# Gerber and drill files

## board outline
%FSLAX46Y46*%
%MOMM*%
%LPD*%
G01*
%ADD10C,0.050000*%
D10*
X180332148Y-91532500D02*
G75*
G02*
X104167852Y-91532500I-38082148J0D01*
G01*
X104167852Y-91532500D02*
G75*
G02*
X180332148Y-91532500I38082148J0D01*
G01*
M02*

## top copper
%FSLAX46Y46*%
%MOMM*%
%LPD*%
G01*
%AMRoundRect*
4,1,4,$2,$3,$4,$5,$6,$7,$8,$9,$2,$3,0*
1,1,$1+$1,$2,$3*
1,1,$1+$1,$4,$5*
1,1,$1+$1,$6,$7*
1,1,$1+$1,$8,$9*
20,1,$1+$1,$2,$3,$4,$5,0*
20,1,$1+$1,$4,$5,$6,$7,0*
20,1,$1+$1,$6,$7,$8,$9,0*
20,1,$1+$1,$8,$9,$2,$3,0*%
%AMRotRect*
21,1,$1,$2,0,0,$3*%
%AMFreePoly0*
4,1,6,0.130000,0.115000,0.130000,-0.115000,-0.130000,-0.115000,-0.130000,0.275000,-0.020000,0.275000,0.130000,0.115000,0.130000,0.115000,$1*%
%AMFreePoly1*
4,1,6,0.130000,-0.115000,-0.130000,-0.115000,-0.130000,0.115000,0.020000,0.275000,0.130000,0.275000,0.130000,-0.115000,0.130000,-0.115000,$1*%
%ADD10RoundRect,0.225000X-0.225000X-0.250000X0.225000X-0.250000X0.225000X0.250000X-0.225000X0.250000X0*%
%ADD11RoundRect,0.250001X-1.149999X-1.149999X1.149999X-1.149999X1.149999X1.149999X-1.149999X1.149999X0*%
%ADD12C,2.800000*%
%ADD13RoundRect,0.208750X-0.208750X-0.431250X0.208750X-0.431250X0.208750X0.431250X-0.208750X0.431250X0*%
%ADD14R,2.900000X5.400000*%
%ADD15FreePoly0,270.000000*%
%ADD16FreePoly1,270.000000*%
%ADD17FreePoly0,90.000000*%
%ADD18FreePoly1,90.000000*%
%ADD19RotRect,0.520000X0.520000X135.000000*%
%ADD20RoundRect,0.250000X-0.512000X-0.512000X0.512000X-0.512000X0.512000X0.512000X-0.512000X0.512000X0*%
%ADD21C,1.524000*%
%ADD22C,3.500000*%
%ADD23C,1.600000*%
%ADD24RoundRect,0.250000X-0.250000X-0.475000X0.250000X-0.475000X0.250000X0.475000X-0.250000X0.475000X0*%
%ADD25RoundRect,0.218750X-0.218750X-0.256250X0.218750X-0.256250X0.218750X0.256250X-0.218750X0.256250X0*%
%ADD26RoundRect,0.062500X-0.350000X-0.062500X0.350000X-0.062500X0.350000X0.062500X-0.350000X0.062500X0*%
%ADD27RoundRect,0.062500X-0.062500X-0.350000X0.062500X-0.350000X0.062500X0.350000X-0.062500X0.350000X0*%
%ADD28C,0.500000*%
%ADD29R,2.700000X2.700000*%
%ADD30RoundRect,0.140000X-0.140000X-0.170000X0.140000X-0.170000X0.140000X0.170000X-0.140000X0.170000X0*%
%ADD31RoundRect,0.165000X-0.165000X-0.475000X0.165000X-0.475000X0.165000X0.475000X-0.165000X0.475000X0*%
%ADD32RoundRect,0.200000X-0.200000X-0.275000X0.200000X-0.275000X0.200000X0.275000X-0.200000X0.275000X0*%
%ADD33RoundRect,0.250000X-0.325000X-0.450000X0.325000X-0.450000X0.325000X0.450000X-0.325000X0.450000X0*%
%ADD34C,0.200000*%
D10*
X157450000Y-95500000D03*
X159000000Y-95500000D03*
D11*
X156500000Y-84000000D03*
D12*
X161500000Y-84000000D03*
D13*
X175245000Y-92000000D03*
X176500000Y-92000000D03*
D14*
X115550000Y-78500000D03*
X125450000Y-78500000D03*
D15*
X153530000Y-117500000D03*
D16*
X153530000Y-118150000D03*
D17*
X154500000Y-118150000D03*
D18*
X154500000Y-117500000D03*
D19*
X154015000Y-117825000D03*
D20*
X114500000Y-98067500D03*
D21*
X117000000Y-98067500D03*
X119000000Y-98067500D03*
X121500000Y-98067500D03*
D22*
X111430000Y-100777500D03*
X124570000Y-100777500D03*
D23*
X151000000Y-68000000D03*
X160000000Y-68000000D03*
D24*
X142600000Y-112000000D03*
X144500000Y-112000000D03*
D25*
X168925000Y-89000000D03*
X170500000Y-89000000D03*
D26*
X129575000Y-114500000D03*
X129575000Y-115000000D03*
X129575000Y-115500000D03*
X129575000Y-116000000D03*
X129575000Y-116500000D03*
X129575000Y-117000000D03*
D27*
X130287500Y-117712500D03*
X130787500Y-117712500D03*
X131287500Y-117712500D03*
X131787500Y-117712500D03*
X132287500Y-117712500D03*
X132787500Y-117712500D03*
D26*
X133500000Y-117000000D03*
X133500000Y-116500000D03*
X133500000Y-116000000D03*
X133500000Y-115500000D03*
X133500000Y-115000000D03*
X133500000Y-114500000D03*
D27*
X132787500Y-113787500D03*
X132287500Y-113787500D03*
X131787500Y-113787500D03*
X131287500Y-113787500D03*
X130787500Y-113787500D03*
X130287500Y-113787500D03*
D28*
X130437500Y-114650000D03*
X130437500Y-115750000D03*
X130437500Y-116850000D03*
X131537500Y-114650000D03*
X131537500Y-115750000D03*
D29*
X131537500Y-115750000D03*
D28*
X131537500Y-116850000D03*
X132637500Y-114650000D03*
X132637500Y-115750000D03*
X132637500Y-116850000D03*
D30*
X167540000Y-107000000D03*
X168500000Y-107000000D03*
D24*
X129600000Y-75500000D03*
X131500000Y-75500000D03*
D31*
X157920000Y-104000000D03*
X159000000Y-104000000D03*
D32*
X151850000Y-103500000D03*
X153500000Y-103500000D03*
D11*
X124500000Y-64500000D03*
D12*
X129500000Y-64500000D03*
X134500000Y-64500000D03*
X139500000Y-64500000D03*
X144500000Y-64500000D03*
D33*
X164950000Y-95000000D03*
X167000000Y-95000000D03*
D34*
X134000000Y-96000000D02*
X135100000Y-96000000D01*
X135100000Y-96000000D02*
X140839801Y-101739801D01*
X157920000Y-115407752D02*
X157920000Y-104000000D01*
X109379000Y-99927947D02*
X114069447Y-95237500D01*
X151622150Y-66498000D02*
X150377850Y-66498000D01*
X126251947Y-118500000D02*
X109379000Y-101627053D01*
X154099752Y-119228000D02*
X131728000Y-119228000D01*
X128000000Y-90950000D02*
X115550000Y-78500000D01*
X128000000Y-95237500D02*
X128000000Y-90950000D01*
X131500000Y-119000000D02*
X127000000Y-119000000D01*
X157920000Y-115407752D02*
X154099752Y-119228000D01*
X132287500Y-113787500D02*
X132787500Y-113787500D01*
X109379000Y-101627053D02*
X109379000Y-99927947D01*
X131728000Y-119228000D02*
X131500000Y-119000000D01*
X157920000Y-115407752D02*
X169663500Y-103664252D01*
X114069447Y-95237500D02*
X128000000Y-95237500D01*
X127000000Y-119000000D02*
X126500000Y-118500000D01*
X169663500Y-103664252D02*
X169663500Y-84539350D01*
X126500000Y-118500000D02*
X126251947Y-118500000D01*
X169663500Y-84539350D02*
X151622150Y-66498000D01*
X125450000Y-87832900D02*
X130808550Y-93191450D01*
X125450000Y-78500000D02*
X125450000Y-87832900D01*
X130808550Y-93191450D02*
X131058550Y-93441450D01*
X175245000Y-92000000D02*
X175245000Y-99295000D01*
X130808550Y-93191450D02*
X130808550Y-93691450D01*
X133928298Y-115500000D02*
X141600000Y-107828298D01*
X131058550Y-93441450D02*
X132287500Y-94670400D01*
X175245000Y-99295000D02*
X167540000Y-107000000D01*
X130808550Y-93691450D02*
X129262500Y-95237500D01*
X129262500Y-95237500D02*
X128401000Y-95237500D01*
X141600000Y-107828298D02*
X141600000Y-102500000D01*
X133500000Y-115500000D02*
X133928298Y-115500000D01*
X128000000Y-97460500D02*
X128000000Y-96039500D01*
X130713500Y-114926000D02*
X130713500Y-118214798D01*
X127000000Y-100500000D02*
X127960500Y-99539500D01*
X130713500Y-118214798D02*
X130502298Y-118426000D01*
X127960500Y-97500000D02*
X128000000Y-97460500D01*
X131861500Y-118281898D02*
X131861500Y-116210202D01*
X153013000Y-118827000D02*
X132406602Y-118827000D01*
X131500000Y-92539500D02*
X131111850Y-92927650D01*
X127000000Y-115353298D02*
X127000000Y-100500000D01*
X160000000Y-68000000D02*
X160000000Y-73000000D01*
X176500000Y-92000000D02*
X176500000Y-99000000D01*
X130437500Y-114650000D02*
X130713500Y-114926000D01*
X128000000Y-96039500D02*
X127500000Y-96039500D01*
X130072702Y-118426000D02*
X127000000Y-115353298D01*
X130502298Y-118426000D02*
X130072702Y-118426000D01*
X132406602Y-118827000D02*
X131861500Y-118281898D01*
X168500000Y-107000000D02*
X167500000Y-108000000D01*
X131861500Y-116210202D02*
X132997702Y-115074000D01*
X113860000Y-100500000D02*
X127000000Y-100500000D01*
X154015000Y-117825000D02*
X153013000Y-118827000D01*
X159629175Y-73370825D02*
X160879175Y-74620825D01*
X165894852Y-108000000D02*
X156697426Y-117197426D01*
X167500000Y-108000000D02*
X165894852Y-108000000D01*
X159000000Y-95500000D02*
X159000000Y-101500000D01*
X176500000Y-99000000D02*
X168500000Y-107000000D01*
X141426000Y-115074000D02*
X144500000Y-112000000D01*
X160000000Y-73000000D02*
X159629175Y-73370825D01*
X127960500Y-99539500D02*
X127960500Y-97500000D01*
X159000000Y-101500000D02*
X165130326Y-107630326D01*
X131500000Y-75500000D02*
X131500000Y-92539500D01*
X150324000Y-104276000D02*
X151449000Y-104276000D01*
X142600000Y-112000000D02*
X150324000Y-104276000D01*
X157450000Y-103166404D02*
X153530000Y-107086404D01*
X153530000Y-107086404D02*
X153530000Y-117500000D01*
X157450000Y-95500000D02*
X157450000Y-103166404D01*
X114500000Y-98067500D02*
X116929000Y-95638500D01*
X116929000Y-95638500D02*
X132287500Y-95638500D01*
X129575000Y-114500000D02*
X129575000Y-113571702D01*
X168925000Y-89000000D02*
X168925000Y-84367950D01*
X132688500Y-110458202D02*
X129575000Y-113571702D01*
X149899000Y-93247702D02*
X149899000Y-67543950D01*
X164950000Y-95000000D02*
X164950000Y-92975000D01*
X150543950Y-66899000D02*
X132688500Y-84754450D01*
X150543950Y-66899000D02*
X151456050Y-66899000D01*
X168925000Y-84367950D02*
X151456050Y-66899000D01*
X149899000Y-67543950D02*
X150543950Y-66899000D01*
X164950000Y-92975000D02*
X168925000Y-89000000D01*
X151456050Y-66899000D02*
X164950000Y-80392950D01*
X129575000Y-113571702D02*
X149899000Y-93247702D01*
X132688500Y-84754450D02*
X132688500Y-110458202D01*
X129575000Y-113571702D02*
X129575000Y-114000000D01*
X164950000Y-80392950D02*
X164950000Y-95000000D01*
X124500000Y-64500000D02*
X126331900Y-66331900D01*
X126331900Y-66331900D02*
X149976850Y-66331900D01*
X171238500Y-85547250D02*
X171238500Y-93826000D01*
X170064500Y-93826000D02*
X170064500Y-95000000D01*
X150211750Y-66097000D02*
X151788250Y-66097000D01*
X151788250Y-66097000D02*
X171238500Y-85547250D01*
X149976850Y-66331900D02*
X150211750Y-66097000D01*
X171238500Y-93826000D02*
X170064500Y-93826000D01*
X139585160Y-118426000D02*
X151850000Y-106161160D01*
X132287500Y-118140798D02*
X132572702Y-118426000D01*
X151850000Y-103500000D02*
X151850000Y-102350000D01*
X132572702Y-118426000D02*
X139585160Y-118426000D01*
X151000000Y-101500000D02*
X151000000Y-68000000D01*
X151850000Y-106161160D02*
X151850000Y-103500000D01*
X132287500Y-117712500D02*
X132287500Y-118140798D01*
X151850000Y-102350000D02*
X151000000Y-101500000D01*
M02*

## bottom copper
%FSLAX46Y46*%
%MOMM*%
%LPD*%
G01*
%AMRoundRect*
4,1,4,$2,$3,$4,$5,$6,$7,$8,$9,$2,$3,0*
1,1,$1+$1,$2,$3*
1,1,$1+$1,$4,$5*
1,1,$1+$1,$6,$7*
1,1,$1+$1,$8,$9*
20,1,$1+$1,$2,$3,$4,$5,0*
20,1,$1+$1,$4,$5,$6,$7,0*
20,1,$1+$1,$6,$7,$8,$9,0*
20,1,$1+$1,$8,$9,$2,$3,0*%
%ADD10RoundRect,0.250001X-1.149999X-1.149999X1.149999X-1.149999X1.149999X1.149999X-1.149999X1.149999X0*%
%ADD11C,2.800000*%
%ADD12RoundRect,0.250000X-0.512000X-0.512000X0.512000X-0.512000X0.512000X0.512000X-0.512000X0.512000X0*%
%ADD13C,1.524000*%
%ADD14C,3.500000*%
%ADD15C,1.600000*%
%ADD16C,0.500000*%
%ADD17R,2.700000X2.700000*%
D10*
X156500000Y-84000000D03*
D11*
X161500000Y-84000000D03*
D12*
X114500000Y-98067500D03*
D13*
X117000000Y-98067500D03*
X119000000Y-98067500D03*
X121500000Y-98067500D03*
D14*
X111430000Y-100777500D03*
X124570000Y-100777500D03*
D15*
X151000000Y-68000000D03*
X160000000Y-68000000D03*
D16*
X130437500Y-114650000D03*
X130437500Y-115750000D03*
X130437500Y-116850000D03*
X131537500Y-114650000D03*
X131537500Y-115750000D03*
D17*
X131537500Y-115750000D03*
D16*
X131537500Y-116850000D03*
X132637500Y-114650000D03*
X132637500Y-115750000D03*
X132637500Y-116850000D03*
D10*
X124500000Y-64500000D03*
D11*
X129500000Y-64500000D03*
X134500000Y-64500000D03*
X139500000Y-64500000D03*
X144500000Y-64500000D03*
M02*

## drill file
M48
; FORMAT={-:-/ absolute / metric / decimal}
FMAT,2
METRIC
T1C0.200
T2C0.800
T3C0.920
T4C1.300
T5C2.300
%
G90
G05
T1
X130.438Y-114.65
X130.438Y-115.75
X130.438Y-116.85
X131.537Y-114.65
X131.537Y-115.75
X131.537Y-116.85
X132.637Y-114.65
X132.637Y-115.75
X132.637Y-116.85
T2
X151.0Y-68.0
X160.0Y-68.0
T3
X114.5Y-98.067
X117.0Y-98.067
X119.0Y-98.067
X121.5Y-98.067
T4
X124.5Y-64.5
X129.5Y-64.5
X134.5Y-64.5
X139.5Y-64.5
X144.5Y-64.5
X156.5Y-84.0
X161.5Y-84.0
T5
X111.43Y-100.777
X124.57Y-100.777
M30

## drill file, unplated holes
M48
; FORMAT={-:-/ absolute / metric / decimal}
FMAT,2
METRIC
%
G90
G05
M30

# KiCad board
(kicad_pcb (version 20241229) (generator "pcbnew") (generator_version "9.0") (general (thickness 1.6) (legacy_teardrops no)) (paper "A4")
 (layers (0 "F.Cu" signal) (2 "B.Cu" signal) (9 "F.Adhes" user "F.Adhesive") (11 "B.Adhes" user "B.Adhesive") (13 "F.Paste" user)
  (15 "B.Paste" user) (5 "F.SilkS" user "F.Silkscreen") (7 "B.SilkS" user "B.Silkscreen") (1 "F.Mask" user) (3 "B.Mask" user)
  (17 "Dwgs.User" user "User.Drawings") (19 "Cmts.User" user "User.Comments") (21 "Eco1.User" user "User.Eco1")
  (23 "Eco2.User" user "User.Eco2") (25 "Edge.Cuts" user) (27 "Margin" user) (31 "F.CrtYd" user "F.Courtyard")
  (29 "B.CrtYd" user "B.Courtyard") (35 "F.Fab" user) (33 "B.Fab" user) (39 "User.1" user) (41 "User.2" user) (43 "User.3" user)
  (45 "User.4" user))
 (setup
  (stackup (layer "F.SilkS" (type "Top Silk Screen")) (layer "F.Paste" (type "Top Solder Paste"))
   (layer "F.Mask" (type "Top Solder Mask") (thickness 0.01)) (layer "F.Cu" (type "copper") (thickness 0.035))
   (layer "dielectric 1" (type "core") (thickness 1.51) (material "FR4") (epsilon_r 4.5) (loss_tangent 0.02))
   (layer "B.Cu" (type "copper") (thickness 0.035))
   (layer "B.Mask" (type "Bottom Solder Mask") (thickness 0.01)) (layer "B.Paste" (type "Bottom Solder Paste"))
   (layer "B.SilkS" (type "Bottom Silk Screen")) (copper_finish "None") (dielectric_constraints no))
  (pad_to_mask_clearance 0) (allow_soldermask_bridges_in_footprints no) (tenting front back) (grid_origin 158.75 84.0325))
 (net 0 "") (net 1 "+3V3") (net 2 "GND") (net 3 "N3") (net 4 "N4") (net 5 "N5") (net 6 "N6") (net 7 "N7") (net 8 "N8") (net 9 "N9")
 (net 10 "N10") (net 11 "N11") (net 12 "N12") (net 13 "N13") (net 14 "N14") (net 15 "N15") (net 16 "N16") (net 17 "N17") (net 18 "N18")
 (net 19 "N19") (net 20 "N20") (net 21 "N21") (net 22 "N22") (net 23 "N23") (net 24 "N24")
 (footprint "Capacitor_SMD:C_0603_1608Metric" (layer "F.Cu") (at 158.225 95.5)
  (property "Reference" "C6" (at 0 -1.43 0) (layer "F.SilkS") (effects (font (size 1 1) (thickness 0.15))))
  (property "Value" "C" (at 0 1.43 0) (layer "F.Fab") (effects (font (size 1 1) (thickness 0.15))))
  (pad "1" smd roundrect (at -0.775 0) (size 0.9 0.95) (layers "F.Cu" "F.Mask" "F.Paste") (roundrect_rratio 0.25) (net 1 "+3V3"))
  (pad "2" smd roundrect (at 0.775 0) (size 0.9 0.95) (layers "F.Cu" "F.Mask" "F.Paste") (roundrect_rratio 0.25) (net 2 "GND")))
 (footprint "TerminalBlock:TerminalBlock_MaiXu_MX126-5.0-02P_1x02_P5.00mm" (layer "F.Cu") (at 156.5 84)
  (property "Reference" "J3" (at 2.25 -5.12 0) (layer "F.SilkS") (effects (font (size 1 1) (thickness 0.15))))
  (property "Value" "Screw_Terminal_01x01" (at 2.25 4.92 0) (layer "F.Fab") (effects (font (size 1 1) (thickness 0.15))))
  (pad "1" thru_hole roundrect (at 0 0) (size 2.8 2.8) (drill 1.3) (layers "*.Cu" "*.Mask") (remove_unused_layers no)
   (roundrect_rratio 0.089286) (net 2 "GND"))
  (pad "2" thru_hole circle (at 5 0) (size 2.8 2.8) (drill 1.3) (layers "*.Cu" "*.Mask") (remove_unused_layers no)))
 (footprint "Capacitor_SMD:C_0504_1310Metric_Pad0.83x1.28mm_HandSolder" (layer "F.Cu") (at 175.8725 92)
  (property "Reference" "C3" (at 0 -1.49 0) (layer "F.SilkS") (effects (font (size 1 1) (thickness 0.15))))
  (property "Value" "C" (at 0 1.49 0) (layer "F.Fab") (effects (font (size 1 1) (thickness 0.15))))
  (pad "1" smd roundrect (at -0.6275 0) (size 0.835 1.28) (layers "F.Cu" "F.Mask" "F.Paste") (roundrect_rratio 0.25) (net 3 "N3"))
  (pad "2" smd roundrect (at 0.6275 0) (size 0.835 1.28) (layers "F.Cu" "F.Mask" "F.Paste") (roundrect_rratio 0.25) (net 2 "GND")))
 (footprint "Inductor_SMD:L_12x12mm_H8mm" (layer "F.Cu") (at 120.5 78.5)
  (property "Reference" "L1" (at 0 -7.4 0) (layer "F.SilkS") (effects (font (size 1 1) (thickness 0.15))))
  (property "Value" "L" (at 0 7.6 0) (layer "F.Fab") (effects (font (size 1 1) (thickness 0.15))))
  (pad "1" smd rect (at -4.95 0) (size 2.9 5.4) (layers "F.Cu" "F.Mask" "F.Paste") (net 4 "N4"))
  (pad "2" smd rect (at 4.95 0) (size 2.9 5.4) (layers "F.Cu" "F.Mask" "F.Paste") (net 3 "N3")))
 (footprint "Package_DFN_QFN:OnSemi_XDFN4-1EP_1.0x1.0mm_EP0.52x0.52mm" (layer "F.Cu") (at 154.015 117.825)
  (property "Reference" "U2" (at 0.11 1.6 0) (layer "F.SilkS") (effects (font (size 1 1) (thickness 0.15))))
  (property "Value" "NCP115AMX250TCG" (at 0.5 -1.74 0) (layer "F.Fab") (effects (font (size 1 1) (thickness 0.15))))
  (pad "1" smd custom (at -0.485 -0.325 270) (size 0.26 0.23) (layers "F.Cu" "F.Mask" "F.Paste") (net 1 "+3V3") (zone_connect 0)
   (thermal_bridge_angle 45) (options (clearance outline) (anchor rect)) (primitives))
  (pad "2" smd custom (at -0.485 0.325 270) (size 0.26 0.23) (layers "F.Cu" "F.Mask" "F.Paste") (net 2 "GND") (zone_connect 0)
   (thermal_bridge_angle 45) (options (clearance outline) (anchor rect)) (primitives))
  (pad "3" smd custom (at 0.485 0.325 90) (size 0.26 0.23) (layers "F.Cu" "F.Mask" "F.Paste") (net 3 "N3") (zone_connect 0)
   (thermal_bridge_angle 45) (options (clearance outline) (anchor rect)) (primitives))
  (pad "4" smd custom (at 0.485 -0.325 90) (size 0.26 0.23) (layers "F.Cu" "F.Mask" "F.Paste") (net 3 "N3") (zone_connect 0)
   (thermal_bridge_angle 45) (options (clearance outline) (anchor rect)) (primitives))
  (pad "5" smd rect (at 0 0 135) (size 0.52 0.52) (layers "F.Cu" "F.Mask" "F.Paste") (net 2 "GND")))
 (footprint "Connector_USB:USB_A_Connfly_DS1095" (layer "F.Cu") (at 114.5 98.0675)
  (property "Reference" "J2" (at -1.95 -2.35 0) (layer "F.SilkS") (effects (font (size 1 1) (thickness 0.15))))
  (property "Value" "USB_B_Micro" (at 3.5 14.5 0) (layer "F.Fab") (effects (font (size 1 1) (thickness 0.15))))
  (pad "1" thru_hole roundrect (at 0 0) (size 1.524 1.524) (drill 0.92) (layers "*.Cu" "*.Mask") (remove_unused_layers no)
   (roundrect_rratio 0.1640419948) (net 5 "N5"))
  (pad "2" thru_hole circle (at 2.5 0) (size 1.524 1.524) (drill 0.92) (layers "*.Cu" "*.Mask") (remove_unused_layers no) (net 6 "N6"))
  (pad "3" thru_hole circle (at 4.5 0) (size 1.524 1.524) (drill 0.92) (layers "*.Cu" "*.Mask") (remove_unused_layers no) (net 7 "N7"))
  (pad "4" thru_hole circle (at 7 0) (size 1.524 1.524) (drill 0.92) (layers "*.Cu" "*.Mask") (remove_unused_layers no) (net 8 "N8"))
  (pad "5" thru_hole circle (at -3.07 2.71) (size 3.5 3.5) (drill 2.3) (layers "*.Cu" "*.Mask") (remove_unused_layers no) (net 2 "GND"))
  (pad "5" thru_hole circle (at 10.07 2.71) (size 3.5 3.5) (drill 2.3) (layers "*.Cu" "*.Mask") (remove_unused_layers no) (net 2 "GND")))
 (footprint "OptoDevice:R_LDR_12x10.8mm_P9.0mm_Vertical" (layer "F.Cu") (at 151 68)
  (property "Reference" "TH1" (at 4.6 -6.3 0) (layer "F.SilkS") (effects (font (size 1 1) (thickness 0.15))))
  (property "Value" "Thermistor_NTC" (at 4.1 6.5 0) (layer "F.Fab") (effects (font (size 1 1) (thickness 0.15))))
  (pad "1" thru_hole circle (at 0 0) (size 1.6 1.6) (drill 0.8) (layers "*.Cu" "*.Mask") (remove_unused_layers no) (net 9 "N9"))
  (pad "2" thru_hole circle (at 9 0) (size 1.6 1.6) (drill 0.8) (layers "*.Cu" "*.Mask") (remove_unused_layers no) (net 2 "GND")))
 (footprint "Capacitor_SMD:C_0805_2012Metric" (layer "F.Cu") (at 143.55 112)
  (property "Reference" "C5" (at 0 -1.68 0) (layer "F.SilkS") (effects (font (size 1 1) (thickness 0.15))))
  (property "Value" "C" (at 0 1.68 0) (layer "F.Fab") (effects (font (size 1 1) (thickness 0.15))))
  (pad "1" smd roundrect (at -0.95 0) (size 1 1.45) (layers "F.Cu" "F.Mask" "F.Paste") (roundrect_rratio 0.25) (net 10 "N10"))
  (pad "2" smd roundrect (at 0.95 0) (size 1 1.45) (layers "F.Cu" "F.Mask" "F.Paste") (roundrect_rratio 0.25) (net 2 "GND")))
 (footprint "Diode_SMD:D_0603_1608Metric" (layer "F.Cu") (at 169.7125 89)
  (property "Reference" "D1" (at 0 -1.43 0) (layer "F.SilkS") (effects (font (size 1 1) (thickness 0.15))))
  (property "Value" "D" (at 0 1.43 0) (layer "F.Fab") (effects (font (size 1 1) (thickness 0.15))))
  (pad "1" smd roundrect (at -0.7875 0) (size 0.875 0.95) (layers "F.Cu" "F.Mask" "F.Paste") (roundrect_rratio 0.25) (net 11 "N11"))
  (pad "2" smd roundrect (at 0.7875 0) (size 0.875 0.95) (layers "F.Cu" "F.Mask" "F.Paste") (roundrect_rratio 0.25) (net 5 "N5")))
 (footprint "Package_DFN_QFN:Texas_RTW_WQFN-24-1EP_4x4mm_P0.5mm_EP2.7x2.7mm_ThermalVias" (layer "F.Cu") (at 131.5375 115.75)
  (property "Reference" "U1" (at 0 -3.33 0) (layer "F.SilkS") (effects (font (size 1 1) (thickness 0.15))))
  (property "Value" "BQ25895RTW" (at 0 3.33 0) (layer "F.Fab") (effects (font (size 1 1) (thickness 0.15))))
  (pad "" smd roundrect (at -0.675 -0.675) (size 1.13 1.13) (layers "F.Paste") (roundrect_rratio 0.221239))
  (pad "" smd roundrect (at -0.675 0.675) (size 1.13 1.13) (layers "F.Paste") (roundrect_rratio 0.221239))
  (pad "" smd roundrect (at 0.675 -0.675) (size 1.13 1.13) (layers "F.Paste") (roundrect_rratio 0.221239))
  (pad "" smd roundrect (at 0.675 0.675) (size 1.13 1.13) (layers "F.Paste") (roundrect_rratio 0.221239))
  (pad "1" smd roundrect (at -1.9625 -1.25) (size 0.825 0.25) (layers "F.Cu" "F.Mask" "F.Paste") (roundrect_rratio 0.25) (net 11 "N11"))
  (pad "2" smd roundrect (at -1.9625 -0.75) (size 0.825 0.25) (layers "F.Cu" "F.Mask" "F.Paste") (roundrect_rratio 0.25) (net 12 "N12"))
  (pad "3" smd roundrect (at -1.9625 -0.25) (size 0.825 0.25) (layers "F.Cu" "F.Mask" "F.Paste") (roundrect_rratio 0.25) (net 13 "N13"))
  (pad "4" smd roundrect (at -1.9625 0.25) (size 0.825 0.25) (layers "F.Cu" "F.Mask" "F.Paste") (roundrect_rratio 0.25) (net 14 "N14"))
  (pad "5" smd roundrect (at -1.9625 0.75) (size 0.825 0.25) (layers "F.Cu" "F.Mask" "F.Paste") (roundrect_rratio 0.25) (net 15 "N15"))
  (pad "6" smd roundrect (at -1.9625 1.25) (size 0.825 0.25) (layers "F.Cu" "F.Mask" "F.Paste") (roundrect_rratio 0.25) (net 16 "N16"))
  (pad "7" smd roundrect (at -1.25 1.9625) (size 0.25 0.825) (layers "F.Cu" "F.Mask" "F.Paste") (roundrect_rratio 0.25) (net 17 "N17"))
  (pad "8" smd roundrect (at -0.75 1.9625) (size 0.25 0.825) (layers "F.Cu" "F.Mask" "F.Paste") (roundrect_rratio 0.25) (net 2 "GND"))
  (pad "9" smd roundrect (at -0.25 1.9625) (size 0.25 0.825) (layers "F.Cu" "F.Mask" "F.Paste") (roundrect_rratio 0.25) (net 2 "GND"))
  (pad "10" smd roundrect (at 0.25 1.9625) (size 0.25 0.825) (layers "F.Cu" "F.Mask" "F.Paste") (roundrect_rratio 0.25) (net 2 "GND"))
  (pad "11" smd roundrect (at 0.75 1.9625) (size 0.25 0.825) (layers "F.Cu" "F.Mask" "F.Paste") (roundrect_rratio 0.25) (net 9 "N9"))
  (pad "12" smd roundrect (at 1.25 1.9625) (size 0.25 0.825) (layers "F.Cu" "F.Mask" "F.Paste") (roundrect_rratio 0.25) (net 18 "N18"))
  (pad "13" smd roundrect (at 1.9625 1.25) (size 0.825 0.25) (layers "F.Cu" "F.Mask" "F.Paste") (roundrect_rratio 0.25) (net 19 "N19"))
  (pad "14" smd roundrect (at 1.9625 0.75) (size 0.825 0.25) (layers "F.Cu" "F.Mask" "F.Paste") (roundrect_rratio 0.25) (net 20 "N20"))
  (pad "15" smd roundrect (at 1.9625 0.25) (size 0.825 0.25) (layers "F.Cu" "F.Mask" "F.Paste") (roundrect_rratio 0.25) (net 3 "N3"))
  (pad "16" smd roundrect (at 1.9625 -0.25) (size 0.825 0.25) (layers "F.Cu" "F.Mask" "F.Paste") (roundrect_rratio 0.25) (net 3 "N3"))
  (pad "17" smd roundrect (at 1.9625 -0.75) (size 0.825 0.25) (layers "F.Cu" "F.Mask" "F.Paste") (roundrect_rratio 0.25) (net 2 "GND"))
  (pad "18" smd roundrect (at 1.9625 -1.25) (size 0.825 0.25) (layers "F.Cu" "F.Mask" "F.Paste") (roundrect_rratio 0.25) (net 2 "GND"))
  (pad "19" smd roundrect (at 1.25 -1.9625) (size 0.25 0.825) (layers "F.Cu" "F.Mask" "F.Paste") (roundrect_rratio 0.25) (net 4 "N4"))
  (pad "20" smd roundrect (at 0.75 -1.9625) (size 0.25 0.825) (layers "F.Cu" "F.Mask" "F.Paste") (roundrect_rratio 0.25) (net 4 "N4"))
  (pad "21" smd roundrect (at 0.25 -1.9625) (size 0.25 0.825) (layers "F.Cu" "F.Mask" "F.Paste") (roundrect_rratio 0.25) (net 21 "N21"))
  (pad "22" smd roundrect (at -0.25 -1.9625) (size 0.25 0.825) (layers "F.Cu" "F.Mask" "F.Paste") (roundrect_rratio 0.25) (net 10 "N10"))
  (pad "23" smd roundrect (at -0.75 -1.9625) (size 0.25 0.825) (layers "F.Cu" "F.Mask" "F.Paste") (roundrect_rratio 0.25) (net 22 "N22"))
  (pad "24" smd roundrect (at -1.25 -1.9625) (size 0.25 0.825) (layers "F.Cu" "F.Mask" "F.Paste") (roundrect_rratio 0.25) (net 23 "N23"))
  (pad "25" thru_hole circle (at -1.1 -1.1) (size 0.5 0.5) (drill 0.2) (layers "*.Cu") (remove_unused_layers no) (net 2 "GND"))
  (pad "25" thru_hole circle (at -1.1 0) (size 0.5 0.5) (drill 0.2) (layers "*.Cu") (remove_unused_layers no) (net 2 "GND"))
  (pad "25" thru_hole circle (at -1.1 1.1) (size 0.5 0.5) (drill 0.2) (layers "*.Cu") (remove_unused_layers no) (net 2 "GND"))
  (pad "25" thru_hole circle (at 0 -1.1) (size 0.5 0.5) (drill 0.2) (layers "*.Cu") (remove_unused_layers no) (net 2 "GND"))
  (pad "25" thru_hole circle (at 0 0) (size 0.5 0.5) (drill 0.2) (layers "*.Cu") (remove_unused_layers no) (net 2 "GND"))
  (pad "25" smd rect (at 0 0) (size 2.7 2.7) (layers "F.Cu" "F.Mask") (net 2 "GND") (zone_connect 2))
  (pad "25" smd rect (at 0 0) (size 2.7 2.7) (layers "B.Cu") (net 2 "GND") (zone_connect 2))
  (pad "25" thru_hole circle (at 0 1.1) (size 0.5 0.5) (drill 0.2) (layers "*.Cu") (remove_unused_layers no) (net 2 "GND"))
  (pad "25" thru_hole circle (at 1.1 -1.1) (size 0.5 0.5) (drill 0.2) (layers "*.Cu") (remove_unused_layers no) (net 2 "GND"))
  (pad "25" thru_hole circle (at 1.1 0) (size 0.5 0.5) (drill 0.2) (layers "*.Cu") (remove_unused_layers no) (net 2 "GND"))
  (pad "25" thru_hole circle (at 1.1 1.1) (size 0.5 0.5) (drill 0.2) (layers "*.Cu") (remove_unused_layers no) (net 2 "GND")))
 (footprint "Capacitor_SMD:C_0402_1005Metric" (layer "F.Cu") (at 168.02 107)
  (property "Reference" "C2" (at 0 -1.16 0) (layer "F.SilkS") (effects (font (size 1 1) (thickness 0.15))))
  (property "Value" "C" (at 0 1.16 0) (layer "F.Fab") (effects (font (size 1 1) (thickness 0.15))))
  (pad "1" smd roundrect (at -0.48 0) (size 0.56 0.62) (layers "F.Cu" "F.Mask" "F.Paste") (roundrect_rratio 0.25) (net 3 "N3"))
  (pad "2" smd roundrect (at 0.48 0) (size 0.56 0.62) (layers "F.Cu" "F.Mask" "F.Paste") (roundrect_rratio 0.25) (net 2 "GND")))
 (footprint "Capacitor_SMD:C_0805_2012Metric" (layer "F.Cu") (at 130.55 75.5)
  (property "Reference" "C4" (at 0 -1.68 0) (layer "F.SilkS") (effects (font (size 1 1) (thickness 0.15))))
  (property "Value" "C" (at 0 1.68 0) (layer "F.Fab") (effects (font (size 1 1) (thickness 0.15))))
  (pad "1" smd roundrect (at -0.95 0) (size 1 1.45) (layers "F.Cu" "F.Mask" "F.Paste") (roundrect_rratio 0.25) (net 3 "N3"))
  (pad "2" smd roundrect (at 0.95 0) (size 1 1.45) (layers "F.Cu" "F.Mask" "F.Paste") (roundrect_rratio 0.25) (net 2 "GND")))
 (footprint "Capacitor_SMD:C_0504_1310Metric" (layer "F.Cu") (at 158.46 104)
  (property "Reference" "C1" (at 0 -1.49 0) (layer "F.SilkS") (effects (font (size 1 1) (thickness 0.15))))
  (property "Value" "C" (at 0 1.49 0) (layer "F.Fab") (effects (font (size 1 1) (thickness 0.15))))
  (pad "1" smd roundrect (at -0.54 0) (size 0.66 1.28) (layers "F.Cu" "F.Mask" "F.Paste") (roundrect_rratio 0.25) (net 4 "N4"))
  (pad "2" smd roundrect (at 0.54 0) (size 0.66 1.28) (layers "F.Cu" "F.Mask" "F.Paste") (roundrect_rratio 0.25) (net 21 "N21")))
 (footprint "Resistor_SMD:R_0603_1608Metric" (layer "F.Cu") (at 152.675 103.5)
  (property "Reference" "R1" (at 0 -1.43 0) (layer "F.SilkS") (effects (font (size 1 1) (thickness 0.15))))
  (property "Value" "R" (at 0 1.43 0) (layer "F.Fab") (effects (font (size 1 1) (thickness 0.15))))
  (pad "1" smd roundrect (at -0.825 0) (size 0.8 0.95) (layers "F.Cu" "F.Mask" "F.Paste") (roundrect_rratio 0.25) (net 9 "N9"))
  (pad "2" smd roundrect (at 0.825 0) (size 0.8 0.95) (layers "F.Cu" "F.Mask" "F.Paste") (roundrect_rratio 0.25) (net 10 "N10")))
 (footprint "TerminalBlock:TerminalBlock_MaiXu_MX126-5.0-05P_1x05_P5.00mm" (layer "F.Cu") (at 124.5 64.5)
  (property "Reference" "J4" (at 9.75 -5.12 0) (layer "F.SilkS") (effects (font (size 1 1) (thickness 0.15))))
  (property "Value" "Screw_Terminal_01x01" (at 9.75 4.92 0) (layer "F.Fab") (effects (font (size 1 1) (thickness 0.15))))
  (pad "1" thru_hole roundrect (at 0 0) (size 2.8 2.8) (drill 1.3) (layers "*.Cu" "*.Mask") (remove_unused_layers no)
   (roundrect_rratio 0.089286) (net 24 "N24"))
  (pad "2" thru_hole circle (at 5 0) (size 2.8 2.8) (drill 1.3) (layers "*.Cu" "*.Mask") (remove_unused_layers no))
  (pad "3" thru_hole circle (at 10 0) (size 2.8 2.8) (drill 1.3) (layers "*.Cu" "*.Mask") (remove_unused_layers no))
  (pad "4" thru_hole circle (at 15 0) (size 2.8 2.8) (drill 1.3) (layers "*.Cu" "*.Mask") (remove_unused_layers no))
  (pad "5" thru_hole circle (at 20 0) (size 2.8 2.8) (drill 1.3) (layers "*.Cu" "*.Mask") (remove_unused_layers no)))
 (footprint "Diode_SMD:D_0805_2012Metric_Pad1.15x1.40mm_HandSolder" (layer "F.Cu") (at 165.975 95)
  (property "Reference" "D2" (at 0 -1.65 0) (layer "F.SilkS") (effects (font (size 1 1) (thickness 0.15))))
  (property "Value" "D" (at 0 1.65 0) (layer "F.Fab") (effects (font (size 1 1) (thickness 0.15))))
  (pad "1" smd roundrect (at -1.025 0) (size 1.15 1.4) (layers "F.Cu" "F.Mask" "F.Paste") (roundrect_rratio 0.217391) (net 11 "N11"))
  (pad "2" smd roundrect (at 1.025 0) (size 1.15 1.4) (layers "F.Cu" "F.Mask" "F.Paste") (roundrect_rratio 0.217391) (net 24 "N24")))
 (gr_circle (center 142.25 91.5325) (end 144.75 129.5325) (stroke (width 0.05) (type default)) (fill no) (layer "Edge.Cuts"))
 (segment (start 134 96) (end 135.1 96) (width 0.2) (layer "F.Cu") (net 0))
 (segment (start 135.1 96) (end 140.839801 101.739801) (width 0.2) (layer "F.Cu") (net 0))
 (segment (start 157.92 115.407752) (end 157.92 104) (width 0.2) (layer "F.Cu") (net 4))
 (segment (start 109.379 99.927947) (end 114.069447 95.2375) (width 0.2) (layer "F.Cu") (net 4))
 (segment (start 151.62215 66.498) (end 150.37785 66.498) (width 0.2) (layer "F.Cu") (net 4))
 (segment (start 126.251947 118.5) (end 109.379 101.627053) (width 0.2) (layer "F.Cu") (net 4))
 (segment (start 154.099752 119.228) (end 131.728 119.228) (width 0.2) (layer "F.Cu") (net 4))
 (segment (start 128 90.95) (end 115.55 78.5) (width 0.2) (layer "F.Cu") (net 4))
 (segment (start 128 95.2375) (end 128 90.95) (width 0.2) (layer "F.Cu") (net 4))
 (segment (start 131.5 119) (end 127 119) (width 0.2) (layer "F.Cu") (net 4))
 (segment (start 157.92 115.407752) (end 154.099752 119.228) (width 0.2) (layer "F.Cu") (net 4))
 (segment (start 132.2875 113.7875) (end 132.7875 113.7875) (width 0.2) (layer "F.Cu") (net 4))
 (segment (start 109.379 101.627053) (end 109.379 99.927947) (width 0.2) (layer "F.Cu") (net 4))
 (segment (start 131.728 119.228) (end 131.5 119) (width 0.2) (layer "F.Cu") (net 4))
 (segment (start 157.92 115.407752) (end 169.6635 103.664252) (width 0.2) (layer "F.Cu") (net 4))
 (segment (start 114.069447 95.2375) (end 128 95.2375) (width 0.2) (layer "F.Cu") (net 4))
 (segment (start 127 119) (end 126.5 118.5) (width 0.2) (layer "F.Cu") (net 4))
 (segment (start 169.6635 103.664252) (end 169.6635 84.53935) (width 0.2) (layer "F.Cu") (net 4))
 (segment (start 126.5 118.5) (end 126.251947 118.5) (width 0.2) (layer "F.Cu") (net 4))
 (segment (start 169.6635 84.53935) (end 151.62215 66.498) (width 0.2) (layer "F.Cu") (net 4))
 (segment (start 125.45 87.8329) (end 130.80855 93.19145) (width 0.2) (layer "F.Cu") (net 3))
 (segment (start 125.45 78.5) (end 125.45 87.8329) (width 0.2) (layer "F.Cu") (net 3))
 (segment (start 130.80855 93.19145) (end 131.05855 93.44145) (width 0.2) (layer "F.Cu") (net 3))
 (segment (start 175.245 92) (end 175.245 99.295) (width 0.2) (layer "F.Cu") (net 3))
 (segment (start 130.80855 93.19145) (end 130.80855 93.69145) (width 0.2) (layer "F.Cu") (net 3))
 (segment (start 133.928298 115.5) (end 141.6 107.828298) (width 0.2) (layer "F.Cu") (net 3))
 (segment (start 131.05855 93.44145) (end 132.2875 94.6704) (width 0.2) (layer "F.Cu") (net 3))
 (segment (start 175.245 99.295) (end 167.54 107) (width 0.2) (layer "F.Cu") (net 3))
 (segment (start 130.80855 93.69145) (end 129.2625 95.2375) (width 0.2) (layer "F.Cu") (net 3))
 (segment (start 129.2625 95.2375) (end 128.401 95.2375) (width 0.2) (layer "F.Cu") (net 3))
 (segment (start 141.6 107.828298) (end 141.6 102.5) (width 0.2) (layer "F.Cu") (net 3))
 (segment (start 133.5 115.5) (end 133.928298 115.5) (width 0.2) (layer "F.Cu") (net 3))
 (segment (start 128 97.4605) (end 128 96.0395) (width 0.2) (layer "F.Cu") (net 2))
 (segment (start 130.7135 114.926) (end 130.7135 118.214798) (width 0.2) (layer "F.Cu") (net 2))
 (segment (start 127 100.5) (end 127.9605 99.5395) (width 0.2) (layer "F.Cu") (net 2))
 (segment (start 130.7135 118.214798) (end 130.502298 118.426) (width 0.2) (layer "F.Cu") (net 2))
 (segment (start 127.9605 97.5) (end 128 97.4605) (width 0.2) (layer "F.Cu") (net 2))
 (segment (start 131.8615 118.281898) (end 131.8615 116.210202) (width 0.2) (layer "F.Cu") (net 2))
 (segment (start 153.013 118.827) (end 132.406602 118.827) (width 0.2) (layer "F.Cu") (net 2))
 (segment (start 131.5 92.5395) (end 131.11185 92.92765) (width 0.2) (layer "F.Cu") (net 2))
 (segment (start 127 115.353298) (end 127 100.5) (width 0.2) (layer "F.Cu") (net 2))
 (segment (start 160 68) (end 160 73) (width 0.2) (layer "F.Cu") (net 2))
 (segment (start 176.5 92) (end 176.5 99) (width 0.2) (layer "F.Cu") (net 2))
 (segment (start 130.4375 114.65) (end 130.7135 114.926) (width 0.2) (layer "F.Cu") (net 2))
 (segment (start 128 96.0395) (end 127.5 96.0395) (width 0.2) (layer "F.Cu") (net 2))
 (segment (start 130.072702 118.426) (end 127 115.353298) (width 0.2) (layer "F.Cu") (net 2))
 (segment (start 130.502298 118.426) (end 130.072702 118.426) (width 0.2) (layer "F.Cu") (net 2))
 (segment (start 132.406602 118.827) (end 131.8615 118.281898) (width 0.2) (layer "F.Cu") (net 2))
 (segment (start 168.5 107) (end 167.5 108) (width 0.2) (layer "F.Cu") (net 2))
 (segment (start 131.8615 116.210202) (end 132.997702 115.074) (width 0.2) (layer "F.Cu") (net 2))
 (segment (start 113.86 100.5) (end 127 100.5) (width 0.2) (layer "F.Cu") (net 2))
 (segment (start 154.015 117.825) (end 153.013 118.827) (width 0.2) (layer "F.Cu") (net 2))
 (segment (start 159.629175 73.370825) (end 160.879175 74.620825) (width 0.2) (layer "F.Cu") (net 2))
 (segment (start 165.894852 108) (end 156.697426 117.197426) (width 0.2) (layer "F.Cu") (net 2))
 (segment (start 167.5 108) (end 165.894852 108) (width 0.2) (layer "F.Cu") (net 2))
 (segment (start 159 95.5) (end 159 101.5) (width 0.2) (layer "F.Cu") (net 2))
 (segment (start 176.5 99) (end 168.5 107) (width 0.2) (layer "F.Cu") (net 2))
 (segment (start 141.426 115.074) (end 144.5 112) (width 0.2) (layer "F.Cu") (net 2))
 (segment (start 160 73) (end 159.629175 73.370825) (width 0.2) (layer "F.Cu") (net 2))
 (segment (start 127.9605 99.5395) (end 127.9605 97.5) (width 0.2) (layer "F.Cu") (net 2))
 (segment (start 159 101.5) (end 165.130326 107.630326) (width 0.2) (layer "F.Cu") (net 2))
 (segment (start 131.5 75.5) (end 131.5 92.5395) (width 0.2) (layer "F.Cu") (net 2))
 (segment (start 150.324 104.276) (end 151.449 104.276) (width 0.2) (layer "F.Cu") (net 10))
 (segment (start 142.6 112) (end 150.324 104.276) (width 0.2) (layer "F.Cu") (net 10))
 (segment (start 157.45 103.166404) (end 153.53 107.086404) (width 0.2) (layer "F.Cu") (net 1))
 (segment (start 153.53 107.086404) (end 153.53 117.5) (width 0.2) (layer "F.Cu") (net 1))
 (segment (start 157.45 95.5) (end 157.45 103.166404) (width 0.2) (layer "F.Cu") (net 1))
 (segment (start 114.5 98.0675) (end 116.929 95.6385) (width 0.2) (layer "F.Cu") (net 5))
 (segment (start 116.929 95.6385) (end 132.2875 95.6385) (width 0.2) (layer "F.Cu") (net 5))
 (segment (start 129.575 114.5) (end 129.575 113.571702) (width 0.2) (layer "F.Cu") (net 11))
 (segment (start 168.925 89) (end 168.925 84.36795) (width 0.2) (layer "F.Cu") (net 11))
 (segment (start 132.6885 110.458202) (end 129.575 113.571702) (width 0.2) (layer "F.Cu") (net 11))
 (segment (start 149.899 93.247702) (end 149.899 67.54395) (width 0.2) (layer "F.Cu") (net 11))
 (segment (start 164.95 95) (end 164.95 92.975) (width 0.2) (layer "F.Cu") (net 11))
 (segment (start 150.54395 66.899) (end 132.6885 84.75445) (width 0.2) (layer "F.Cu") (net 11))
 (segment (start 150.54395 66.899) (end 151.45605 66.899) (width 0.2) (layer "F.Cu") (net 11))
 (segment (start 168.925 84.36795) (end 151.45605 66.899) (width 0.2) (layer "F.Cu") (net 11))
 (segment (start 149.899 67.54395) (end 150.54395 66.899) (width 0.2) (layer "F.Cu") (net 11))
 (segment (start 164.95 92.975) (end 168.925 89) (width 0.2) (layer "F.Cu") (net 11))
 (segment (start 151.45605 66.899) (end 164.95 80.39295) (width 0.2) (layer "F.Cu") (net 11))
 (segment (start 129.575 113.571702) (end 149.899 93.247702) (width 0.2) (layer "F.Cu") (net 11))
 (segment (start 132.6885 84.75445) (end 132.6885 110.458202) (width 0.2) (layer "F.Cu") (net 11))
 (segment (start 129.575 113.571702) (end 129.575 114) (width 0.2) (layer "F.Cu") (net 11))
 (segment (start 164.95 80.39295) (end 164.95 95) (width 0.2) (layer "F.Cu") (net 11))
 (segment (start 124.5 64.5) (end 126.3319 66.3319) (width 0.2) (layer "F.Cu") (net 24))
 (segment (start 126.3319 66.3319) (end 149.97685 66.3319) (width 0.2) (layer "F.Cu") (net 24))
 (segment (start 171.2385 85.54725) (end 171.2385 93.826) (width 0.2) (layer "F.Cu") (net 24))
 (segment (start 170.0645 93.826) (end 170.0645 95) (width 0.2) (layer "F.Cu") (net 24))
 (segment (start 150.21175 66.097) (end 151.78825 66.097) (width 0.2) (layer "F.Cu") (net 24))
 (segment (start 151.78825 66.097) (end 171.2385 85.54725) (width 0.2) (layer "F.Cu") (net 24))
 (segment (start 149.97685 66.3319) (end 150.21175 66.097) (width 0.2) (layer "F.Cu") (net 24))
 (segment (start 171.2385 93.826) (end 170.0645 93.826) (width 0.2) (layer "F.Cu") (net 24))
 (segment (start 139.58516 118.426) (end 151.85 106.16116) (width 0.2) (layer "F.Cu") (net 9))
 (segment (start 132.2875 118.140798) (end 132.572702 118.426) (width 0.2) (layer "F.Cu") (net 9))
 (segment (start 151.85 103.5) (end 151.85 102.35) (width 0.2) (layer "F.Cu") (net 9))
 (segment (start 132.572702 118.426) (end 139.58516 118.426) (width 0.2) (layer "F.Cu") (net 9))
 (segment (start 151 101.5) (end 151 68) (width 0.2) (layer "F.Cu") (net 9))
 (segment (start 151.85 106.16116) (end 151.85 103.5) (width 0.2) (layer "F.Cu") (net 9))
 (segment (start 132.2875 117.7125) (end 132.2875 118.140798) (width 0.2) (layer "F.Cu") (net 9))
 (segment (start 151.85 102.35) (end 151 101.5) (width 0.2) (layer "F.Cu") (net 9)))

